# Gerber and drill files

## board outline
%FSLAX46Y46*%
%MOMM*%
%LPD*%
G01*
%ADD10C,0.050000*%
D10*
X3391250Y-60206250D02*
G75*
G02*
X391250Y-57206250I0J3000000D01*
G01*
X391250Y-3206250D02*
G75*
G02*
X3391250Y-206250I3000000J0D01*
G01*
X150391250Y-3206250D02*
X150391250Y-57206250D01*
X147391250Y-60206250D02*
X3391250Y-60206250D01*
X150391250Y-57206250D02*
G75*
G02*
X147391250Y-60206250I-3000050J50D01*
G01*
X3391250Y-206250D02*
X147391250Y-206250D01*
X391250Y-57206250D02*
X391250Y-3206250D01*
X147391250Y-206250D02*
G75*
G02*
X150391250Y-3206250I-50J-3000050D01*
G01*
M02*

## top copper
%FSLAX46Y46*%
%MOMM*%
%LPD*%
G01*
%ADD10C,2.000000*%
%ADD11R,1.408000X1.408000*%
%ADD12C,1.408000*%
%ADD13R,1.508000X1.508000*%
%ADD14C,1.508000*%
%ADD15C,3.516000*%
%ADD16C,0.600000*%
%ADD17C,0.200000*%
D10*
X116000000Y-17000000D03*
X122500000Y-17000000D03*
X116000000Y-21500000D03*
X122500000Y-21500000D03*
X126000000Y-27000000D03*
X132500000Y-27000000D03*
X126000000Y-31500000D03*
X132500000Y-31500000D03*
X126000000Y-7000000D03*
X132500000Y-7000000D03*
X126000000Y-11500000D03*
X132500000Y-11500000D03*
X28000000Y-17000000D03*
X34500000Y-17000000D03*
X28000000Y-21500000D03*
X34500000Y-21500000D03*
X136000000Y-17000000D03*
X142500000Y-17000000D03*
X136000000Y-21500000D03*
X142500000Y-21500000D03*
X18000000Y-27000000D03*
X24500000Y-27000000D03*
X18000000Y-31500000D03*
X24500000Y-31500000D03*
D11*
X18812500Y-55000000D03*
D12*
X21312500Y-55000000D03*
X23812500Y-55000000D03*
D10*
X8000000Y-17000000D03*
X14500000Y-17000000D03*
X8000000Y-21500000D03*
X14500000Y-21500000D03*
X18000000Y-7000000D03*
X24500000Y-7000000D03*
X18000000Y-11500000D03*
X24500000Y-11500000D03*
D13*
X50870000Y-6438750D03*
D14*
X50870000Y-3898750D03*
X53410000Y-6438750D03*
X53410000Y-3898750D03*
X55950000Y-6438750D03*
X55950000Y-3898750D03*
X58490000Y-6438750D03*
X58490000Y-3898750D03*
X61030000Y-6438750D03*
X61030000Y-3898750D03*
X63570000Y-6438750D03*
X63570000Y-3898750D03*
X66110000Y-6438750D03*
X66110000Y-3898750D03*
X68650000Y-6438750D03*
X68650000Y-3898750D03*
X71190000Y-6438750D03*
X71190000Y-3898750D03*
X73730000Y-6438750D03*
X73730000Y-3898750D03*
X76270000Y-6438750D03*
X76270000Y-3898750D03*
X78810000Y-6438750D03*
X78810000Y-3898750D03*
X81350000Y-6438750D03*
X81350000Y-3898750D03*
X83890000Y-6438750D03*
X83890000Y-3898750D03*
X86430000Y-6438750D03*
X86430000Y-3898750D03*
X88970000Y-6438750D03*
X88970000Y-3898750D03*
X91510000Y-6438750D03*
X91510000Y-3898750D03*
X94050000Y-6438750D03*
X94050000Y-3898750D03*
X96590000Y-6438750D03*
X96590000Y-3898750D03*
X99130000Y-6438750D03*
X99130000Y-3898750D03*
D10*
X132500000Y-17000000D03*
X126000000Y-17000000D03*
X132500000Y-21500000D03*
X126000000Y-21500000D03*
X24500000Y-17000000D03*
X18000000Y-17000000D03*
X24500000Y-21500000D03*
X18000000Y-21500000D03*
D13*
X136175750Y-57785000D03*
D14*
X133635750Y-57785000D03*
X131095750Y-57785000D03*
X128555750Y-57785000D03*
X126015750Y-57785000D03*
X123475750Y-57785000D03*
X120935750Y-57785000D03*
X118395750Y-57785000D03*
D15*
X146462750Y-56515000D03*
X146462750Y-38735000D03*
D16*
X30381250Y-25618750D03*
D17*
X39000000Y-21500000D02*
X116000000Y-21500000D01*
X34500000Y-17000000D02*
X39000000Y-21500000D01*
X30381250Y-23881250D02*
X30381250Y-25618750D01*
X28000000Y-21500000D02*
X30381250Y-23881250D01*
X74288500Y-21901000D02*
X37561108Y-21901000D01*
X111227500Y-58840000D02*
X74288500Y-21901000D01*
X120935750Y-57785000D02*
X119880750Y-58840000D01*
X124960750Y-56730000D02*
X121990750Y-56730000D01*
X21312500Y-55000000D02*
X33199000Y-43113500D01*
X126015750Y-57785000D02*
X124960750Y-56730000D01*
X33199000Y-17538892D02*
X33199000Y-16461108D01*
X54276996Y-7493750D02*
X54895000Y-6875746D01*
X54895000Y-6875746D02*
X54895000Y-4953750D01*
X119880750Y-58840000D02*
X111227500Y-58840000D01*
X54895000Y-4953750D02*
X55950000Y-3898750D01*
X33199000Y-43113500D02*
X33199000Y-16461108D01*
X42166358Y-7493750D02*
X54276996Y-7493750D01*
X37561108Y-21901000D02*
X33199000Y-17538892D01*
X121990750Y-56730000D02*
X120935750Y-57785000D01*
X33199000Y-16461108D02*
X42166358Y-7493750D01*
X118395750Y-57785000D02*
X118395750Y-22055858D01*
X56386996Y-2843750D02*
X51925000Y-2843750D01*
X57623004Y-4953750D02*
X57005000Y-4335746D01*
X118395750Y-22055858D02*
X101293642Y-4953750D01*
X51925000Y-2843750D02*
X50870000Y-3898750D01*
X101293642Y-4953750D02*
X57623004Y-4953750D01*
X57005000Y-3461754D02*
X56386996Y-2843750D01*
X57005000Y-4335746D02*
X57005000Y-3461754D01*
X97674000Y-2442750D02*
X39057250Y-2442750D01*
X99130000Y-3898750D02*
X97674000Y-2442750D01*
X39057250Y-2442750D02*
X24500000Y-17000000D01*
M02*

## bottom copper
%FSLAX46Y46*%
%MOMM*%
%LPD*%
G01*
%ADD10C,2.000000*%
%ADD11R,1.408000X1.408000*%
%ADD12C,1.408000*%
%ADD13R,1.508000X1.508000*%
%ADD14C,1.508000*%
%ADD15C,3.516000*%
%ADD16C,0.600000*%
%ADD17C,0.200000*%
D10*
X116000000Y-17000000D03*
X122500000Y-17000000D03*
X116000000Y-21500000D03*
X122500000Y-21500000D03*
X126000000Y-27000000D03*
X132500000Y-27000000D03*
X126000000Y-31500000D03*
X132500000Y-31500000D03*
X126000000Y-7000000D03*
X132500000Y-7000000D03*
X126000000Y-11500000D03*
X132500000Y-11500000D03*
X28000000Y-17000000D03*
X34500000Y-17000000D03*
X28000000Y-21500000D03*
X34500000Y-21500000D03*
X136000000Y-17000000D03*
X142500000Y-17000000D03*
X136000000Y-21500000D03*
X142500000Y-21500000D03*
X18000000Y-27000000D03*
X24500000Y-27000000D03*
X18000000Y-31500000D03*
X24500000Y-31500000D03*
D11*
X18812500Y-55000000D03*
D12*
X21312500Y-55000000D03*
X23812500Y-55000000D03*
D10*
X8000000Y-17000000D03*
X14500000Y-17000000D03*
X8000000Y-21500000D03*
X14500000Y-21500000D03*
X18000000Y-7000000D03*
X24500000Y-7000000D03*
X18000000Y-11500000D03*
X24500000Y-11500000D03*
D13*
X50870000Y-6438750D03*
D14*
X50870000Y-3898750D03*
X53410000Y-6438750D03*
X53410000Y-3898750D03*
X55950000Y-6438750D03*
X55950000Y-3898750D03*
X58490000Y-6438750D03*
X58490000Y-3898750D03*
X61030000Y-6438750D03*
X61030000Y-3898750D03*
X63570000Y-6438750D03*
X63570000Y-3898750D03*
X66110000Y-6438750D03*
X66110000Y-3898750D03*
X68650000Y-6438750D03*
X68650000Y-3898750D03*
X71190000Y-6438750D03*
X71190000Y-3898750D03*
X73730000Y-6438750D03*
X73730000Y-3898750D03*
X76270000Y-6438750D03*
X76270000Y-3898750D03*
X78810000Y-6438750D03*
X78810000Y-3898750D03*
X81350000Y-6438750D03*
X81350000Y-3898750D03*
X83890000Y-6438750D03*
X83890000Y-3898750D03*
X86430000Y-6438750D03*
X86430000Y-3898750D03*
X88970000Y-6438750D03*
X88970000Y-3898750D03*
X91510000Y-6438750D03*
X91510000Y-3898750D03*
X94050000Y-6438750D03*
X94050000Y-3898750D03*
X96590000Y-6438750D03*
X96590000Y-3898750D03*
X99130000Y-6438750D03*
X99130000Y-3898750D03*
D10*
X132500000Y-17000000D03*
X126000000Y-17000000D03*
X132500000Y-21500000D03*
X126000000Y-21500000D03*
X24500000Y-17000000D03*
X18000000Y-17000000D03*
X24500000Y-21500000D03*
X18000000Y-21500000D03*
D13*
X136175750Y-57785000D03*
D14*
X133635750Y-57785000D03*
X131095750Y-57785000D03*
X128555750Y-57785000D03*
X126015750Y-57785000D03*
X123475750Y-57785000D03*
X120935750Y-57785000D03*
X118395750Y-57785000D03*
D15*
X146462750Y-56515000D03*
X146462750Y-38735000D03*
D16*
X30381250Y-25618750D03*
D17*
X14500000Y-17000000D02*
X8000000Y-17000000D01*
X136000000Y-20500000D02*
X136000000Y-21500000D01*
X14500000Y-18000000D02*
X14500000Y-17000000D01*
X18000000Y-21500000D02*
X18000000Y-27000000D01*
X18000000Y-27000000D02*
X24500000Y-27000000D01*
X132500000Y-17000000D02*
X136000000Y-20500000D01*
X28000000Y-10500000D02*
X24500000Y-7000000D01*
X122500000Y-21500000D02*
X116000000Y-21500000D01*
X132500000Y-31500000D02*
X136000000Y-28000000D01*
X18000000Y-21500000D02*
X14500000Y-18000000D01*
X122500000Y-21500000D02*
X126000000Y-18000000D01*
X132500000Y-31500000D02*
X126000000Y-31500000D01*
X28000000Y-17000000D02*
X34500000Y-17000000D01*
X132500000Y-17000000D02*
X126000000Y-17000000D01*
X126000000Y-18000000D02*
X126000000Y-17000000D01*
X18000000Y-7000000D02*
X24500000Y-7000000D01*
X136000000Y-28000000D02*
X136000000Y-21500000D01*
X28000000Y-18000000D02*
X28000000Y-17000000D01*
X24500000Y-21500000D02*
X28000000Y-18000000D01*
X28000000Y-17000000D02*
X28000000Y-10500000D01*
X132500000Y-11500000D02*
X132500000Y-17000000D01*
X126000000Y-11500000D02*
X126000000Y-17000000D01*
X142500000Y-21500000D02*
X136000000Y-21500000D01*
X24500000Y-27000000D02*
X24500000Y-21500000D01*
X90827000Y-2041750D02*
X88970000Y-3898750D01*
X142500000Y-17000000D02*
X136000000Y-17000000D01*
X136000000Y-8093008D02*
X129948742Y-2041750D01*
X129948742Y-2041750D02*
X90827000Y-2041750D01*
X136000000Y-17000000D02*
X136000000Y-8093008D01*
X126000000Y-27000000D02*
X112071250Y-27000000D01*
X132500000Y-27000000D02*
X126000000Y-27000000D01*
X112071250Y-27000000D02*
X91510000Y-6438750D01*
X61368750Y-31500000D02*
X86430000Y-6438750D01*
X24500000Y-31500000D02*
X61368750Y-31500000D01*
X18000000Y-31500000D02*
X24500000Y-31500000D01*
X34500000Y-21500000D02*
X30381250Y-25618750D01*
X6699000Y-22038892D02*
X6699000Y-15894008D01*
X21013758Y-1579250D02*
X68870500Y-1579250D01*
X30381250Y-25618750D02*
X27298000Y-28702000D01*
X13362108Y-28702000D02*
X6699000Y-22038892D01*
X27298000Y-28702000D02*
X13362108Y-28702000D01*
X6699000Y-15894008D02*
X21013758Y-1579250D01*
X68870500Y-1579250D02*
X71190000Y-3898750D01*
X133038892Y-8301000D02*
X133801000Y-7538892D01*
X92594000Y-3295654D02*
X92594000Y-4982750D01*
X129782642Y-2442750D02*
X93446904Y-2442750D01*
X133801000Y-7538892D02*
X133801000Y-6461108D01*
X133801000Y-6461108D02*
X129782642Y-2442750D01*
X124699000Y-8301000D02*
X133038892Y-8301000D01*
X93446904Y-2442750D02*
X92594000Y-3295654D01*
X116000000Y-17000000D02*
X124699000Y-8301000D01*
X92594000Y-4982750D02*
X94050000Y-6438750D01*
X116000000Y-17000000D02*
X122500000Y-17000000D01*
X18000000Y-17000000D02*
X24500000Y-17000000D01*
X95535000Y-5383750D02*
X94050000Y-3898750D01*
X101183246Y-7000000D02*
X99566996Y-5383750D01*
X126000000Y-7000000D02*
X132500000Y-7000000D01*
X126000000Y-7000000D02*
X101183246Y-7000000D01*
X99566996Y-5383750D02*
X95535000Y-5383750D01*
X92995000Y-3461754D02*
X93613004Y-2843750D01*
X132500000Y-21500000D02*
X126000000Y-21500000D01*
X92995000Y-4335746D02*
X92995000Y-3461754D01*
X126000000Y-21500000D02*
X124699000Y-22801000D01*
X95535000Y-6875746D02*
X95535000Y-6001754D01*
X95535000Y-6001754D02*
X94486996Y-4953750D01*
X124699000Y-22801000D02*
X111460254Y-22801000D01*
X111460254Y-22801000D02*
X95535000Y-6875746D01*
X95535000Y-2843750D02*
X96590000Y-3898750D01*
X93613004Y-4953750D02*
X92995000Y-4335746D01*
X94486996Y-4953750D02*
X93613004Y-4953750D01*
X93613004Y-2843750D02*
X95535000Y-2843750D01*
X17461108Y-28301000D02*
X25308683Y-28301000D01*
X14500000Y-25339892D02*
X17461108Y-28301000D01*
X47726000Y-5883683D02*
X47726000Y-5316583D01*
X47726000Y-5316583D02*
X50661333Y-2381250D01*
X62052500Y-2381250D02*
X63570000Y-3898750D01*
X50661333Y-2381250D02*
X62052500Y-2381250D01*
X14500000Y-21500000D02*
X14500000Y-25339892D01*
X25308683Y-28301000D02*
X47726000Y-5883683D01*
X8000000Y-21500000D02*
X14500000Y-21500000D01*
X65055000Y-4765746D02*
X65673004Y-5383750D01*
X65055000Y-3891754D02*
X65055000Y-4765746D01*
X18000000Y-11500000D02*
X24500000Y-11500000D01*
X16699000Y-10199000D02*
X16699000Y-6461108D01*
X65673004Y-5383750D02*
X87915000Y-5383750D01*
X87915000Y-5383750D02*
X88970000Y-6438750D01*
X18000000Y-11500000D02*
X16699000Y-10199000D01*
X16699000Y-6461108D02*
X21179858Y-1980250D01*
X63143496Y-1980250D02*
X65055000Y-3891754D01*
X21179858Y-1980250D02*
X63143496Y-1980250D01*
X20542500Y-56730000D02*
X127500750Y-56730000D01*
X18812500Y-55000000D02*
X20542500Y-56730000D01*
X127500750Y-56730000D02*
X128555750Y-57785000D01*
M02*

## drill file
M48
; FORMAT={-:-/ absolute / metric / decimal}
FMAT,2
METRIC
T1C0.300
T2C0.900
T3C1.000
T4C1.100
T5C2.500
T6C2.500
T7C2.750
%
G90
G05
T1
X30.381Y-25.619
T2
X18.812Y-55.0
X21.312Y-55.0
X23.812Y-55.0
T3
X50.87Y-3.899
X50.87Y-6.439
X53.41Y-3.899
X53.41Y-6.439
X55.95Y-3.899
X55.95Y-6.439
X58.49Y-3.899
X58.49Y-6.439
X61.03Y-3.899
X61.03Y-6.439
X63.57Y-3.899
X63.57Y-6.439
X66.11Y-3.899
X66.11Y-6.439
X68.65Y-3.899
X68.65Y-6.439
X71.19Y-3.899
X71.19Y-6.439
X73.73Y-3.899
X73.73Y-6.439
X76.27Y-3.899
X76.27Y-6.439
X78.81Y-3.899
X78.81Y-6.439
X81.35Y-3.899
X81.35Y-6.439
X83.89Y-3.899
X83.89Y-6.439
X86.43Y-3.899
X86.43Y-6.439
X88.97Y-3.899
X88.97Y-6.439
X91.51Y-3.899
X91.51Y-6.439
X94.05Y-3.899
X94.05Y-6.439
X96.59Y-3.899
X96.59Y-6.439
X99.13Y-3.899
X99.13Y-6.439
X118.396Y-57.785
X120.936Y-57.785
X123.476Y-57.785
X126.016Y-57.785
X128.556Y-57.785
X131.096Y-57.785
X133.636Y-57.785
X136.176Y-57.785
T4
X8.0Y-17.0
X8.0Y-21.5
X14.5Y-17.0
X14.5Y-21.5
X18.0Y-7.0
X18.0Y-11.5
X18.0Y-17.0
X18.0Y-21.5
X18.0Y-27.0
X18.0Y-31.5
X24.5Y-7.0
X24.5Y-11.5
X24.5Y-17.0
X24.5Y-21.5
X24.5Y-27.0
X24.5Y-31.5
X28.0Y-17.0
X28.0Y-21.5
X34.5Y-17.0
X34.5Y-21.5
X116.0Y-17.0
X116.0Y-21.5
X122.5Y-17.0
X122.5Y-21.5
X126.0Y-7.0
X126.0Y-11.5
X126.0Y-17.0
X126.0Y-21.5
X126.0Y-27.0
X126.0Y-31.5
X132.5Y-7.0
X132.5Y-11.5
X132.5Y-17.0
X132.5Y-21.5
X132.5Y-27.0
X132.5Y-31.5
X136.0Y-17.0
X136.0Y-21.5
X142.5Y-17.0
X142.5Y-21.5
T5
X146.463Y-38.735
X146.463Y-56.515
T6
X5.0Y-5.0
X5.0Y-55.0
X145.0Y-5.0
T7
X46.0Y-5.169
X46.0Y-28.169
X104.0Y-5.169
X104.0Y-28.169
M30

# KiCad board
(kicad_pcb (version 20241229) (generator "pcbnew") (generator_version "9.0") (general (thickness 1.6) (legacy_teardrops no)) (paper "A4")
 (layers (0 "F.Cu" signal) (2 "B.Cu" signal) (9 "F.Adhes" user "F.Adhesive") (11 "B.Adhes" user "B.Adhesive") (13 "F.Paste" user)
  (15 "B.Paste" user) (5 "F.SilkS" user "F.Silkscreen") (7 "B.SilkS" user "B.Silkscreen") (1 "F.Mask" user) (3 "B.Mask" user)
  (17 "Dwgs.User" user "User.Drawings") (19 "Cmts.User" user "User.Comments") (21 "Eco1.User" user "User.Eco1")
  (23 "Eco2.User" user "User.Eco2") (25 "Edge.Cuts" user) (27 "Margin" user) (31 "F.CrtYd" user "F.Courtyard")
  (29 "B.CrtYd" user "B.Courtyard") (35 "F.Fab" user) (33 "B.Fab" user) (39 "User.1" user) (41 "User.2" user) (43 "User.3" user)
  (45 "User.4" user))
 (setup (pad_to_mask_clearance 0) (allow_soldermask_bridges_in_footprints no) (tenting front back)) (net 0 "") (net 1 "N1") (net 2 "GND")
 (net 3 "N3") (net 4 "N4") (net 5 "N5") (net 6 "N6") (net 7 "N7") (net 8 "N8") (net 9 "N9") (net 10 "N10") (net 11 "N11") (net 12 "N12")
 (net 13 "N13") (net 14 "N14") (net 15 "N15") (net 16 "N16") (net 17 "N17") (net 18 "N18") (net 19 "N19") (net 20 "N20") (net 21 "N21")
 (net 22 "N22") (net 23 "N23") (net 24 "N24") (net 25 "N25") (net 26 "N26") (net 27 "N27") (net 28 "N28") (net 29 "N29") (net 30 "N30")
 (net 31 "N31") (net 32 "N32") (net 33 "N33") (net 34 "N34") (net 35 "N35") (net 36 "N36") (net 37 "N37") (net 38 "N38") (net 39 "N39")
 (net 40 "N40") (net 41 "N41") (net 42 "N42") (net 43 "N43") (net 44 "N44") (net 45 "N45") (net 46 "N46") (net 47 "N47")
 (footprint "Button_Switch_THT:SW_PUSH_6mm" (layer "F.Cu") (at 116 17)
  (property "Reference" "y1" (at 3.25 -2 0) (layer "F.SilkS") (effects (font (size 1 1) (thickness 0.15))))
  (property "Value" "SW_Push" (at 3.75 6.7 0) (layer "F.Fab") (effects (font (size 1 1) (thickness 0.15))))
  (pad "1" thru_hole circle (at 0 0 90) (size 2 2) (drill 1.1) (layers "*.Cu" "*.Mask") (remove_unused_layers no) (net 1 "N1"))
  (pad "1" thru_hole circle (at 6.5 0 90) (size 2 2) (drill 1.1) (layers "*.Cu" "*.Mask") (remove_unused_layers no) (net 1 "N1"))
  (pad "2" thru_hole circle (at 0 4.5 90) (size 2 2) (drill 1.1) (layers "*.Cu" "*.Mask") (remove_unused_layers no) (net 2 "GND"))
  (pad "2" thru_hole circle (at 6.5 4.5 90) (size 2 2) (drill 1.1) (layers "*.Cu" "*.Mask") (remove_unused_layers no) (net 2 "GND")))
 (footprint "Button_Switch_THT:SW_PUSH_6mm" (layer "F.Cu") (at 126 27)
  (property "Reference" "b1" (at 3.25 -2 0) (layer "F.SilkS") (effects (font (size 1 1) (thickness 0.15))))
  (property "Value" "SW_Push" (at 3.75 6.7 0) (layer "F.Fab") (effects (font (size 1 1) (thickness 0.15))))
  (pad "1" thru_hole circle (at 0 0 90) (size 2 2) (drill 1.1) (layers "*.Cu" "*.Mask") (remove_unused_layers no) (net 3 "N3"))
  (pad "1" thru_hole circle (at 6.5 0 90) (size 2 2) (drill 1.1) (layers "*.Cu" "*.Mask") (remove_unused_layers no) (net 3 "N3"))
  (pad "2" thru_hole circle (at 0 4.5 90) (size 2 2) (drill 1.1) (layers "*.Cu" "*.Mask") (remove_unused_layers no) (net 2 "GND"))
  (pad "2" thru_hole circle (at 6.5 4.5 90) (size 2 2) (drill 1.1) (layers "*.Cu" "*.Mask") (remove_unused_layers no) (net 2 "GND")))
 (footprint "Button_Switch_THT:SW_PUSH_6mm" (layer "F.Cu") (at 126 7)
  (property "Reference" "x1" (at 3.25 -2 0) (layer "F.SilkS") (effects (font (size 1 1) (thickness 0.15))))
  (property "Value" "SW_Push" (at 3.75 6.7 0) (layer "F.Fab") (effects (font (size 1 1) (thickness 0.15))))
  (pad "1" thru_hole circle (at 0 0 90) (size 2 2) (drill 1.1) (layers "*.Cu" "*.Mask") (remove_unused_layers no) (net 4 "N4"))
  (pad "1" thru_hole circle (at 6.5 0 90) (size 2 2) (drill 1.1) (layers "*.Cu" "*.Mask") (remove_unused_layers no) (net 4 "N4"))
  (pad "2" thru_hole circle (at 0 4.5 90) (size 2 2) (drill 1.1) (layers "*.Cu" "*.Mask") (remove_unused_layers no) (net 2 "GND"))
  (pad "2" thru_hole circle (at 6.5 4.5 90) (size 2 2) (drill 1.1) (layers "*.Cu" "*.Mask") (remove_unused_layers no) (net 2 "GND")))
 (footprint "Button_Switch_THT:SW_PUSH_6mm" (layer "F.Cu") (at 28 17)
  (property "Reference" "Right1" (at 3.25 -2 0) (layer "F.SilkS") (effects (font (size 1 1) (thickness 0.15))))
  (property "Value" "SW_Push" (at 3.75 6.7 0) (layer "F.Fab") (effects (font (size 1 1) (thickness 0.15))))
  (pad "1" thru_hole circle (at 0 0 90) (size 2 2) (drill 1.1) (layers "*.Cu" "*.Mask") (remove_unused_layers no) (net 2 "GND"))
  (pad "1" thru_hole circle (at 6.5 0 90) (size 2 2) (drill 1.1) (layers "*.Cu" "*.Mask") (remove_unused_layers no) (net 2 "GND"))
  (pad "2" thru_hole circle (at 0 4.5 90) (size 2 2) (drill 1.1) (layers "*.Cu" "*.Mask") (remove_unused_layers no) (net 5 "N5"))
  (pad "2" thru_hole circle (at 6.5 4.5 90) (size 2 2) (drill 1.1) (layers "*.Cu" "*.Mask") (remove_unused_layers no) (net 5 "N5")))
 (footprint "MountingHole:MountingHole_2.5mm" (layer "F.Cu") (at 145 5)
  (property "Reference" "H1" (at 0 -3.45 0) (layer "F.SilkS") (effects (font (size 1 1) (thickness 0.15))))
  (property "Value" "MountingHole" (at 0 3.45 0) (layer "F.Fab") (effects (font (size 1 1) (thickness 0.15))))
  (pad "" np_thru_hole circle (at 0 0) (size 2.5 2.5) (drill 2.5) (layers "*.Cu" "*.Mask")))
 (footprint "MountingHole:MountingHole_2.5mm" (layer "F.Cu") (at 5 5)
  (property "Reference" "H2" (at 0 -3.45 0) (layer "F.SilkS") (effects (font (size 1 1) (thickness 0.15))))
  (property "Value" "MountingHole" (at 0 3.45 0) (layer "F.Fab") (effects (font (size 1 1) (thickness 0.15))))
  (pad "" np_thru_hole circle (at 0 0) (size 2.5 2.5) (drill 2.5) (layers "*.Cu" "*.Mask")))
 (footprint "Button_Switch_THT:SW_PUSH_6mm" (layer "F.Cu") (at 136 17)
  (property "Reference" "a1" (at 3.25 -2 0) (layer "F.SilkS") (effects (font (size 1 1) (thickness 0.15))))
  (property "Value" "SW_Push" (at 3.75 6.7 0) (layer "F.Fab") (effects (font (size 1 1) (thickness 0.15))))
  (pad "1" thru_hole circle (at 0 0 90) (size 2 2) (drill 1.1) (layers "*.Cu" "*.Mask") (remove_unused_layers no) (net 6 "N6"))
  (pad "1" thru_hole circle (at 6.5 0 90) (size 2 2) (drill 1.1) (layers "*.Cu" "*.Mask") (remove_unused_layers no) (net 6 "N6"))
  (pad "2" thru_hole circle (at 0 4.5 90) (size 2 2) (drill 1.1) (layers "*.Cu" "*.Mask") (remove_unused_layers no) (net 2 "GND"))
  (pad "2" thru_hole circle (at 6.5 4.5 90) (size 2 2) (drill 1.1) (layers "*.Cu" "*.Mask") (remove_unused_layers no) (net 2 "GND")))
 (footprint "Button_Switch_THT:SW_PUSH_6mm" (layer "F.Cu") (at 18 27)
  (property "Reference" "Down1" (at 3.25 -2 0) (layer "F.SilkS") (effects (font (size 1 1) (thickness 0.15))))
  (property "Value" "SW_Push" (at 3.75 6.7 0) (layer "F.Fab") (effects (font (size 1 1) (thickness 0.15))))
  (pad "1" thru_hole circle (at 0 0 90) (size 2 2) (drill 1.1) (layers "*.Cu" "*.Mask") (remove_unused_layers no) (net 2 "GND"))
  (pad "1" thru_hole circle (at 6.5 0 90) (size 2 2) (drill 1.1) (layers "*.Cu" "*.Mask") (remove_unused_layers no) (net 2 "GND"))
  (pad "2" thru_hole circle (at 0 4.5 90) (size 2 2) (drill 1.1) (layers "*.Cu" "*.Mask") (remove_unused_layers no) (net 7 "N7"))
  (pad "2" thru_hole circle (at 6.5 4.5 90) (size 2 2) (drill 1.1) (layers "*.Cu" "*.Mask") (remove_unused_layers no) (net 7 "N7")))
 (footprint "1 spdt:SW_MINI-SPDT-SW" (layer "F.Cu") (at 21.3125 55)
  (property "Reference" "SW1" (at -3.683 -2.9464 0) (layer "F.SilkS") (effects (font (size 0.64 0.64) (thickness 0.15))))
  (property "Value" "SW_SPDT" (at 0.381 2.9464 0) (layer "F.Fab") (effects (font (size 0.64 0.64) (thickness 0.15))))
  (pad "1" thru_hole rect (at -2.5 0) (size 1.408 1.408) (drill 0.9) (layers "*.Cu" "*.Mask") (remove_unused_layers no) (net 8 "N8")
   (solder_mask_margin 0.102))
  (pad "2" thru_hole circle (at 0 0) (size 1.408 1.408) (drill 0.9) (layers "*.Cu" "*.Mask") (remove_unused_layers no) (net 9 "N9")
   (solder_mask_margin 0.102))
  (pad "3" thru_hole circle (at 2.5 0) (size 1.408 1.408) (drill 0.9) (layers "*.Cu" "*.Mask") (remove_unused_layers no) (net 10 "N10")
   (solder_mask_margin 0.102)))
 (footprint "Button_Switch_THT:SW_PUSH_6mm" (layer "F.Cu") (at 8 17)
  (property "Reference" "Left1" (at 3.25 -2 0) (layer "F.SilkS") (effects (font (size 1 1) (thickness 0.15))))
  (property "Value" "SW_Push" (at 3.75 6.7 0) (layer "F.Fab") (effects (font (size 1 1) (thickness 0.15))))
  (pad "1" thru_hole circle (at 0 0 90) (size 2 2) (drill 1.1) (layers "*.Cu" "*.Mask") (remove_unused_layers no) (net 2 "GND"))
  (pad "1" thru_hole circle (at 6.5 0 90) (size 2 2) (drill 1.1) (layers "*.Cu" "*.Mask") (remove_unused_layers no) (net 2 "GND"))
  (pad "2" thru_hole circle (at 0 4.5 90) (size 2 2) (drill 1.1) (layers "*.Cu" "*.Mask") (remove_unused_layers no) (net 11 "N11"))
  (pad "2" thru_hole circle (at 6.5 4.5 90) (size 2 2) (drill 1.1) (layers "*.Cu" "*.Mask") (remove_unused_layers no) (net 11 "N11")))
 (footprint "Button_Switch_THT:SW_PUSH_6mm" (layer "F.Cu") (at 18 7)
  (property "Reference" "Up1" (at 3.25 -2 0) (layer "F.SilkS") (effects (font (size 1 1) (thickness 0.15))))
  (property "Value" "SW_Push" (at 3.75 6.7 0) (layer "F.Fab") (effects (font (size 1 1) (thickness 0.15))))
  (pad "1" thru_hole circle (at 0 0 90) (size 2 2) (drill 1.1) (layers "*.Cu" "*.Mask") (remove_unused_layers no) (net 2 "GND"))
  (pad "1" thru_hole circle (at 6.5 0 90) (size 2 2) (drill 1.1) (layers "*.Cu" "*.Mask") (remove_unused_layers no) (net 2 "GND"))
  (pad "2" thru_hole circle (at 0 4.5 90) (size 2 2) (drill 1.1) (layers "*.Cu" "*.Mask") (remove_unused_layers no) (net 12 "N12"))
  (pad "2" thru_hole circle (at 6.5 4.5 90) (size 2 2) (drill 1.1) (layers "*.Cu" "*.Mask") (remove_unused_layers no) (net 12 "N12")))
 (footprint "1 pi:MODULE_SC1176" (layer "F.Cu") (at 75 16.66875)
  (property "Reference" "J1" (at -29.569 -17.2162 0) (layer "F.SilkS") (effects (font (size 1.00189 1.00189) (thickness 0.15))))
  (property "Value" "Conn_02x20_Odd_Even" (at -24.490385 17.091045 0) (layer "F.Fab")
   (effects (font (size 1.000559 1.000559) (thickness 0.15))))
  (pad "" np_thru_hole circle (at -29 -11.5) (size 2.75 2.75) (drill 2.75) (layers "*.Cu" "*.Mask"))
  (pad "" np_thru_hole circle (at -29 11.5) (size 2.75 2.75) (drill 2.75) (layers "*.Cu" "*.Mask"))
  (pad "" np_thru_hole circle (at 29 -11.5) (size 2.75 2.75) (drill 2.75) (layers "*.Cu" "*.Mask"))
  (pad "" np_thru_hole circle (at 29 11.5) (size 2.75 2.75) (drill 2.75) (layers "*.Cu" "*.Mask"))
  (pad "1" thru_hole rect (at -24.13 -10.23) (size 1.508 1.508) (drill 1) (layers "*.Cu" "*.Mask") (remove_unused_layers no) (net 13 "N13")
   (solder_mask_margin 0.102))
  (pad "2" thru_hole circle (at -24.13 -12.77) (size 1.508 1.508) (drill 1) (layers "*.Cu" "*.Mask") (remove_unused_layers no)
   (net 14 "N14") (solder_mask_margin 0.102))
  (pad "3" thru_hole circle (at -21.59 -10.23) (size 1.508 1.508) (drill 1) (layers "*.Cu" "*.Mask") (remove_unused_layers no)
   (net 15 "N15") (solder_mask_margin 0.102))
  (pad "4" thru_hole circle (at -21.59 -12.77) (size 1.508 1.508) (drill 1) (layers "*.Cu" "*.Mask") (remove_unused_layers no)
   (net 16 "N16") (solder_mask_margin 0.102))
  (pad "5" thru_hole circle (at -19.05 -10.23) (size 1.508 1.508) (drill 1) (layers "*.Cu" "*.Mask") (remove_unused_layers no)
   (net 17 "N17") (solder_mask_margin 0.102))
  (pad "6" thru_hole circle (at -19.05 -12.77) (size 1.508 1.508) (drill 1) (layers "*.Cu" "*.Mask") (remove_unused_layers no) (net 9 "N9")
   (solder_mask_margin 0.102))
  (pad "7" thru_hole circle (at -16.51 -10.23) (size 1.508 1.508) (drill 1) (layers "*.Cu" "*.Mask") (remove_unused_layers no)
   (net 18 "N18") (solder_mask_margin 0.102))
  (pad "8" thru_hole circle (at -16.51 -12.77) (size 1.508 1.508) (drill 1) (layers "*.Cu" "*.Mask") (remove_unused_layers no)
   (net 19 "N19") (solder_mask_margin 0.102))
  (pad "9" thru_hole circle (at -13.97 -10.23) (size 1.508 1.508) (drill 1) (layers "*.Cu" "*.Mask") (remove_unused_layers no)
   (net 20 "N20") (solder_mask_margin 0.102))
  (pad "10" thru_hole circle (at -13.97 -12.77) (size 1.508 1.508) (drill 1) (layers "*.Cu" "*.Mask") (remove_unused_layers no)
   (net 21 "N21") (solder_mask_margin 0.102))
  (pad "11" thru_hole circle (at -11.43 -10.23) (size 1.508 1.508) (drill 1) (layers "*.Cu" "*.Mask") (remove_unused_layers no)
   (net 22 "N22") (solder_mask_margin 0.102))
  (pad "12" thru_hole circle (at -11.43 -12.77) (size 1.508 1.508) (drill 1) (layers "*.Cu" "*.Mask") (remove_unused_layers no)
   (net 11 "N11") (solder_mask_margin 0.102))
  (pad "13" thru_hole circle (at -8.89 -10.23) (size 1.508 1.508) (drill 1) (layers "*.Cu" "*.Mask") (remove_unused_layers no)
   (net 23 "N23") (solder_mask_margin 0.102))
  (pad "14" thru_hole circle (at -8.89 -12.77) (size 1.508 1.508) (drill 1) (layers "*.Cu" "*.Mask") (remove_unused_layers no)
   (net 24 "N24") (solder_mask_margin 0.102))
  (pad "15" thru_hole circle (at -6.35 -10.23) (size 1.508 1.508) (drill 1) (layers "*.Cu" "*.Mask") (remove_unused_layers no)
   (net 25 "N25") (solder_mask_margin 0.102))
  (pad "16" thru_hole circle (at -6.35 -12.77) (size 1.508 1.508) (drill 1) (layers "*.Cu" "*.Mask") (remove_unused_layers no)
   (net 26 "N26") (solder_mask_margin 0.102))
  (pad "17" thru_hole circle (at -3.81 -10.23) (size 1.508 1.508) (drill 1) (layers "*.Cu" "*.Mask") (remove_unused_layers no)
   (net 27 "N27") (solder_mask_margin 0.102))
  (pad "18" thru_hole circle (at -3.81 -12.77) (size 1.508 1.508) (drill 1) (layers "*.Cu" "*.Mask") (remove_unused_layers no) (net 5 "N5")
   (solder_mask_margin 0.102))
  (pad "19" thru_hole circle (at -1.27 -10.23) (size 1.508 1.508) (drill 1) (layers "*.Cu" "*.Mask") (remove_unused_layers no)
   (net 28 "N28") (solder_mask_margin 0.102))
  (pad "20" thru_hole circle (at -1.27 -12.77) (size 1.508 1.508) (drill 1) (layers "*.Cu" "*.Mask") (remove_unused_layers no)
   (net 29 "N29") (solder_mask_margin 0.102))
  (pad "21" thru_hole circle (at 1.27 -10.23) (size 1.508 1.508) (drill 1) (layers "*.Cu" "*.Mask") (remove_unused_layers no) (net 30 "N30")
   (solder_mask_margin 0.102))
  (pad "22" thru_hole circle (at 1.27 -12.77) (size 1.508 1.508) (drill 1) (layers "*.Cu" "*.Mask") (remove_unused_layers no) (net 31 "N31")
   (solder_mask_margin 0.102))
  (pad "23" thru_hole circle (at 3.81 -10.23) (size 1.508 1.508) (drill 1) (layers "*.Cu" "*.Mask") (remove_unused_layers no) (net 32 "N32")
   (solder_mask_margin 0.102))
  (pad "24" thru_hole circle (at 3.81 -12.77) (size 1.508 1.508) (drill 1) (layers "*.Cu" "*.Mask") (remove_unused_layers no) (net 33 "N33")
   (solder_mask_margin 0.102))
  (pad "25" thru_hole circle (at 6.35 -10.23) (size 1.508 1.508) (drill 1) (layers "*.Cu" "*.Mask") (remove_unused_layers no) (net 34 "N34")
   (solder_mask_margin 0.102))
  (pad "26" thru_hole circle (at 6.35 -12.77) (size 1.508 1.508) (drill 1) (layers "*.Cu" "*.Mask") (remove_unused_layers no) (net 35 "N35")
   (solder_mask_margin 0.102))
  (pad "27" thru_hole circle (at 8.89 -10.23) (size 1.508 1.508) (drill 1) (layers "*.Cu" "*.Mask") (remove_unused_layers no) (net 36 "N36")
   (solder_mask_margin 0.102))
  (pad "28" thru_hole circle (at 8.89 -12.77) (size 1.508 1.508) (drill 1) (layers "*.Cu" "*.Mask") (remove_unused_layers no) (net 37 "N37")
   (solder_mask_margin 0.102))
  (pad "29" thru_hole circle (at 11.43 -10.23) (size 1.508 1.508) (drill 1) (layers "*.Cu" "*.Mask") (remove_unused_layers no) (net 7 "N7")
   (solder_mask_margin 0.102))
  (pad "30" thru_hole circle (at 11.43 -12.77) (size 1.508 1.508) (drill 1) (layers "*.Cu" "*.Mask") (remove_unused_layers no)
   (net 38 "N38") (solder_mask_margin 0.102))
  (pad "31" thru_hole circle (at 13.97 -10.23) (size 1.508 1.508) (drill 1) (layers "*.Cu" "*.Mask") (remove_unused_layers no)
   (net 12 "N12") (solder_mask_margin 0.102))
  (pad "32" thru_hole circle (at 13.97 -12.77) (size 1.508 1.508) (drill 1) (layers "*.Cu" "*.Mask") (remove_unused_layers no) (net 6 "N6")
   (solder_mask_margin 0.102))
  (pad "33" thru_hole circle (at 16.51 -10.23) (size 1.508 1.508) (drill 1) (layers "*.Cu" "*.Mask") (remove_unused_layers no) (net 3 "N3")
   (solder_mask_margin 0.102))
  (pad "34" thru_hole circle (at 16.51 -12.77) (size 1.508 1.508) (drill 1) (layers "*.Cu" "*.Mask") (remove_unused_layers no)
   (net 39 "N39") (solder_mask_margin 0.102))
  (pad "35" thru_hole circle (at 19.05 -10.23) (size 1.508 1.508) (drill 1) (layers "*.Cu" "*.Mask") (remove_unused_layers no) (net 1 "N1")
   (solder_mask_margin 0.102))
  (pad "36" thru_hole circle (at 19.05 -12.77) (size 1.508 1.508) (drill 1) (layers "*.Cu" "*.Mask") (remove_unused_layers no) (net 4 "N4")
   (solder_mask_margin 0.102))
  (pad "37" thru_hole circle (at 21.59 -10.23) (size 1.508 1.508) (drill 1) (layers "*.Cu" "*.Mask") (remove_unused_layers no)
   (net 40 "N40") (solder_mask_margin 0.102))
  (pad "38" thru_hole circle (at 21.59 -12.77) (size 1.508 1.508) (drill 1) (layers "*.Cu" "*.Mask") (remove_unused_layers no)
   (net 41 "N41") (solder_mask_margin 0.102))
  (pad "39" thru_hole circle (at 24.13 -10.23) (size 1.508 1.508) (drill 1) (layers "*.Cu" "*.Mask") (remove_unused_layers no)
   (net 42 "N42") (solder_mask_margin 0.102))
  (pad "40" thru_hole circle (at 24.13 -12.77) (size 1.508 1.508) (drill 1) (layers "*.Cu" "*.Mask") (remove_unused_layers no)
   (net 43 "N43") (solder_mask_margin 0.102)))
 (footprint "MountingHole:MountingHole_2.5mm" (layer "F.Cu") (at 5 55)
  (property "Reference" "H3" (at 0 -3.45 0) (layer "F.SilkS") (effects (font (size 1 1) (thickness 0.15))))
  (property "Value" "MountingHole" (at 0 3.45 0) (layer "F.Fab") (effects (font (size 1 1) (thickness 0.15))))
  (pad "" np_thru_hole circle (at 0 0) (size 2.5 2.5) (drill 2.5) (layers "*.Cu" "*.Mask")))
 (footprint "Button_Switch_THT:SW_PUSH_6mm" (layer "B.Cu") (at 132.5 17 180)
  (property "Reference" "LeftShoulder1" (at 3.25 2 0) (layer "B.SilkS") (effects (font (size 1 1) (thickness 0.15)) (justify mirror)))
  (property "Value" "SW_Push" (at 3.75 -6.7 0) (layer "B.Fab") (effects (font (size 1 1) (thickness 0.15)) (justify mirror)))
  (pad "1" thru_hole circle (at 0 0 90) (size 2 2) (drill 1.1) (layers "*.Cu" "*.Mask") (remove_unused_layers no) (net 2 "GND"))
  (pad "1" thru_hole circle (at 6.5 0 90) (size 2 2) (drill 1.1) (layers "*.Cu" "*.Mask") (remove_unused_layers no) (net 2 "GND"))
  (pad "2" thru_hole circle (at 0 -4.5 90) (size 2 2) (drill 1.1) (layers "*.Cu" "*.Mask") (remove_unused_layers no) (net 41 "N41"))
  (pad "2" thru_hole circle (at 6.5 -4.5 90) (size 2 2) (drill 1.1) (layers "*.Cu" "*.Mask") (remove_unused_layers no) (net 41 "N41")))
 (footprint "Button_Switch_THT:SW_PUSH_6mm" (layer "B.Cu") (at 24.5 17 180)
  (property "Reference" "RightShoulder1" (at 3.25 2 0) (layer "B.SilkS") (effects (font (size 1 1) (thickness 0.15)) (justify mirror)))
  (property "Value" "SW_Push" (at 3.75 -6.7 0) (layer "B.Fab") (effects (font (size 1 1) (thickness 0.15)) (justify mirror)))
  (pad "1" thru_hole circle (at 0 0 90) (size 2 2) (drill 1.1) (layers "*.Cu" "*.Mask") (remove_unused_layers no) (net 43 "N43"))
  (pad "1" thru_hole circle (at 6.5 0 90) (size 2 2) (drill 1.1) (layers "*.Cu" "*.Mask") (remove_unused_layers no) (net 43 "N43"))
  (pad "2" thru_hole circle (at 0 -4.5 90) (size 2 2) (drill 1.1) (layers "*.Cu" "*.Mask") (remove_unused_layers no) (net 2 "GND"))
  (pad "2" thru_hole circle (at 6.5 -4.5 90) (size 2 2) (drill 1.1) (layers "*.Cu" "*.Mask") (remove_unused_layers no) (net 2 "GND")))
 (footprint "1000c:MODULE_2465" (layer "B.Cu") (at 130.96875 47.625 180)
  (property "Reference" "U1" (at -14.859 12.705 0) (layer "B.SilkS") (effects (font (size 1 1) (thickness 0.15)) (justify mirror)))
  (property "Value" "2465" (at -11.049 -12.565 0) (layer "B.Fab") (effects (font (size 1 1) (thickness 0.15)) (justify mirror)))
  (pad "1" thru_hole rect (at -5.207 -10.16 180) (size 1.508 1.508) (drill 1) (layers "*.Cu" "*.Mask") (remove_unused_layers no)
   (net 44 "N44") (solder_mask_margin 0.102))
  (pad "2" thru_hole circle (at -2.667 -10.16 180) (size 1.508 1.508) (drill 1) (layers "*.Cu" "*.Mask") (remove_unused_layers no)
   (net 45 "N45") (solder_mask_margin 0.102))
  (pad "3" thru_hole circle (at -0.127 -10.16 180) (size 1.508 1.508) (drill 1) (layers "*.Cu" "*.Mask") (remove_unused_layers no)
   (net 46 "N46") (solder_mask_margin 0.102))
  (pad "4" thru_hole circle (at 2.413 -10.16 180) (size 1.508 1.508) (drill 1) (layers "*.Cu" "*.Mask") (remove_unused_layers no)
   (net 8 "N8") (solder_mask_margin 0.102))
  (pad "5" thru_hole circle (at 4.953 -10.16 180) (size 1.508 1.508) (drill 1) (layers "*.Cu" "*.Mask") (remove_unused_layers no)
   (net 9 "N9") (solder_mask_margin 0.102))
  (pad "6" thru_hole circle (at 7.493 -10.16 180) (size 1.508 1.508) (drill 1) (layers "*.Cu" "*.Mask") (remove_unused_layers no)
   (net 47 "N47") (solder_mask_margin 0.102))
  (pad "7" thru_hole circle (at 10.033 -10.16 180) (size 1.508 1.508) (drill 1) (layers "*.Cu" "*.Mask") (remove_unused_layers no)
   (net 9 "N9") (solder_mask_margin 0.102))
  (pad "8" thru_hole circle (at 12.573 -10.16 180) (size 1.508 1.508) (drill 1) (layers "*.Cu" "*.Mask") (remove_unused_layers no)
   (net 14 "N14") (solder_mask_margin 0.102))
  (pad "P1" thru_hole circle (at -15.494 -8.89 180) (size 3.516 3.516) (drill 2.5) (layers "*.Cu" "*.Mask") (remove_unused_layers no)
   (solder_mask_margin 0.102))
  (pad "P2" thru_hole circle (at -15.494 8.89 180) (size 3.516 3.516) (drill 2.5) (layers "*.Cu" "*.Mask") (remove_unused_layers no)
   (solder_mask_margin 0.102)))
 (gr_arc (start 3.39125 60.20625) (mid 1.26993 59.32757) (end 0.39125 57.20625) (stroke (width 0.05) (type default)) (layer "Edge.Cuts"))
 (gr_arc (start 0.39125 3.20625) (mid 1.26993 1.08493) (end 3.39125 0.20625) (stroke (width 0.05) (type default)) (layer "Edge.Cuts"))
 (gr_line (start 150.39125 3.20625) (end 150.39125 57.20625) (stroke (width 0.05) (type default)) (layer "Edge.Cuts"))
 (gr_line (start 147.39125 60.20625) (end 3.39125 60.20625) (stroke (width 0.05) (type default)) (layer "Edge.Cuts"))
 (gr_arc (start 150.39125 57.20625) (mid 149.51257 59.32757) (end 147.39125 60.20625) (stroke (width 0.05) (type default))
  (layer "Edge.Cuts"))
 (gr_line (start 3.39125 0.20625) (end 147.39125 0.20625) (stroke (width 0.05) (type default)) (layer "Edge.Cuts"))
 (gr_line (start 0.39125 57.20625) (end 0.39125 3.20625) (stroke (width 0.05) (type default)) (layer "Edge.Cuts"))
 (gr_arc (start 147.39125 0.20625) (mid 149.51257 1.08493) (end 150.39125 3.20625) (stroke (width 0.05) (type default)) (layer "Edge.Cuts"))
 (segment (start 39 21.5) (end 116 21.5) (width 0.2) (layer "F.Cu") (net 2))
 (segment (start 34.5 17) (end 39 21.5) (width 0.2) (layer "F.Cu") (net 2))
 (segment (start 14.5 17) (end 8 17) (width 0.2) (layer "B.Cu") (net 2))
 (segment (start 136 20.5) (end 136 21.5) (width 0.2) (layer "B.Cu") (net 2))
 (segment (start 14.5 18) (end 14.5 17) (width 0.2) (layer "B.Cu") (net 2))
 (segment (start 18 21.5) (end 18 27) (width 0.2) (layer "B.Cu") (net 2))
 (segment (start 18 27) (end 24.5 27) (width 0.2) (layer "B.Cu") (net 2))
 (segment (start 132.5 17) (end 136 20.5) (width 0.2) (layer "B.Cu") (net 2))
 (segment (start 28 10.5) (end 24.5 7) (width 0.2) (layer "B.Cu") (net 2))
 (segment (start 122.5 21.5) (end 116 21.5) (width 0.2) (layer "B.Cu") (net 2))
 (segment (start 132.5 31.5) (end 136 28) (width 0.2) (layer "B.Cu") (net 2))
 (segment (start 18 21.5) (end 14.5 18) (width 0.2) (layer "B.Cu") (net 2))
 (segment (start 122.5 21.5) (end 126 18) (width 0.2) (layer "B.Cu") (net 2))
 (segment (start 132.5 31.5) (end 126 31.5) (width 0.2) (layer "B.Cu") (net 2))
 (segment (start 28 17) (end 34.5 17) (width 0.2) (layer "B.Cu") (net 2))
 (segment (start 132.5 17) (end 126 17) (width 0.2) (layer "B.Cu") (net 2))
 (segment (start 126 18) (end 126 17) (width 0.2) (layer "B.Cu") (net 2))
 (segment (start 18 7) (end 24.5 7) (width 0.2) (layer "B.Cu") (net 2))
 (segment (start 136 28) (end 136 21.5) (width 0.2) (layer "B.Cu") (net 2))
 (segment (start 28 18) (end 28 17) (width 0.2) (layer "B.Cu") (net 2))
 (segment (start 24.5 21.5) (end 28 18) (width 0.2) (layer "B.Cu") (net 2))
 (segment (start 28 17) (end 28 10.5) (width 0.2) (layer "B.Cu") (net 2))
 (segment (start 132.5 11.5) (end 132.5 17) (width 0.2) (layer "B.Cu") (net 2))
 (segment (start 126 11.5) (end 126 17) (width 0.2) (layer "B.Cu") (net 2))
 (segment (start 142.5 21.5) (end 136 21.5) (width 0.2) (layer "B.Cu") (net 2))
 (segment (start 24.5 27) (end 24.5 21.5) (width 0.2) (layer "B.Cu") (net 2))
 (segment (start 90.827 2.04175) (end 88.97 3.89875) (width 0.2) (layer "B.Cu") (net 6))
 (segment (start 142.5 17) (end 136 17) (width 0.2) (layer "B.Cu") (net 6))
 (segment (start 136 8.093008) (end 129.948742 2.04175) (width 0.2) (layer "B.Cu") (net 6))
 (segment (start 129.948742 2.04175) (end 90.827 2.04175) (width 0.2) (layer "B.Cu") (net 6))
 (segment (start 136 17) (end 136 8.093008) (width 0.2) (layer "B.Cu") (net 6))
 (segment (start 126 27) (end 112.07125 27) (width 0.2) (layer "B.Cu") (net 3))
 (segment (start 132.5 27) (end 126 27) (width 0.2) (layer "B.Cu") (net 3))
 (segment (start 112.07125 27) (end 91.51 6.43875) (width 0.2) (layer "B.Cu") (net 3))
 (segment (start 61.36875 31.5) (end 86.43 6.43875) (width 0.2) (layer "B.Cu") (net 7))
 (segment (start 24.5 31.5) (end 61.36875 31.5) (width 0.2) (layer "B.Cu") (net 7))
 (segment (start 18 31.5) (end 24.5 31.5) (width 0.2) (layer "B.Cu") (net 7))
 (segment (start 30.38125 23.88125) (end 30.38125 25.61875) (width 0.2) (layer "F.Cu") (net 5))
 (segment (start 28 21.5) (end 30.38125 23.88125) (width 0.2) (layer "F.Cu") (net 5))
 (via (at 30.38125 25.61875) (size 0.6) (drill 0.3) (layers "F.Cu" "B.Cu") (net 5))
 (segment (start 34.5 21.5) (end 30.38125 25.61875) (width 0.2) (layer "B.Cu") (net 5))
 (segment (start 6.699 22.038892) (end 6.699 15.894008) (width 0.2) (layer "B.Cu") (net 5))
 (segment (start 21.013758 1.57925) (end 68.8705 1.57925) (width 0.2) (layer "B.Cu") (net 5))
 (segment (start 30.38125 25.61875) (end 27.298 28.702) (width 0.2) (layer "B.Cu") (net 5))
 (segment (start 13.362108 28.702) (end 6.699 22.038892) (width 0.2) (layer "B.Cu") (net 5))
 (segment (start 27.298 28.702) (end 13.362108 28.702) (width 0.2) (layer "B.Cu") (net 5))
 (segment (start 6.699 15.894008) (end 21.013758 1.57925) (width 0.2) (layer "B.Cu") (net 5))
 (segment (start 68.8705 1.57925) (end 71.19 3.89875) (width 0.2) (layer "B.Cu") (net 5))
 (segment (start 74.2885 21.901) (end 37.561108 21.901) (width 0.2) (layer "F.Cu") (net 9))
 (segment (start 111.2275 58.84) (end 74.2885 21.901) (width 0.2) (layer "F.Cu") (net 9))
 (segment (start 120.93575 57.785) (end 119.88075 58.84) (width 0.2) (layer "F.Cu") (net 9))
 (segment (start 124.96075 56.73) (end 121.99075 56.73) (width 0.2) (layer "F.Cu") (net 9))
 (segment (start 21.3125 55) (end 33.199 43.1135) (width 0.2) (layer "F.Cu") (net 9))
 (segment (start 126.01575 57.785) (end 124.96075 56.73) (width 0.2) (layer "F.Cu") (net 9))
 (segment (start 33.199 17.538892) (end 33.199 16.461108) (width 0.2) (layer "F.Cu") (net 9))
 (segment (start 54.276996 7.49375) (end 54.895 6.875746) (width 0.2) (layer "F.Cu") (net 9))
 (segment (start 54.895 6.875746) (end 54.895 4.95375) (width 0.2) (layer "F.Cu") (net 9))
 (segment (start 119.88075 58.84) (end 111.2275 58.84) (width 0.2) (layer "F.Cu") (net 9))
 (segment (start 54.895 4.95375) (end 55.95 3.89875) (width 0.2) (layer "F.Cu") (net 9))
 (segment (start 33.199 43.1135) (end 33.199 16.461108) (width 0.2) (layer "F.Cu") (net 9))
 (segment (start 42.166358 7.49375) (end 54.276996 7.49375) (width 0.2) (layer "F.Cu") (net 9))
 (segment (start 37.561108 21.901) (end 33.199 17.538892) (width 0.2) (layer "F.Cu") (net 9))
 (segment (start 121.99075 56.73) (end 120.93575 57.785) (width 0.2) (layer "F.Cu") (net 9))
 (segment (start 33.199 16.461108) (end 42.166358 7.49375) (width 0.2) (layer "F.Cu") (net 9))
 (segment (start 133.038892 8.301) (end 133.801 7.538892) (width 0.2) (layer "B.Cu") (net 1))
 (segment (start 92.594 3.295654) (end 92.594 4.98275) (width 0.2) (layer "B.Cu") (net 1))
 (segment (start 129.782642 2.44275) (end 93.446904 2.44275) (width 0.2) (layer "B.Cu") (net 1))
 (segment (start 133.801 7.538892) (end 133.801 6.461108) (width 0.2) (layer "B.Cu") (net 1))
 (segment (start 133.801 6.461108) (end 129.782642 2.44275) (width 0.2) (layer "B.Cu") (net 1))
 (segment (start 124.699 8.301) (end 133.038892 8.301) (width 0.2) (layer "B.Cu") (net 1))
 (segment (start 93.446904 2.44275) (end 92.594 3.295654) (width 0.2) (layer "B.Cu") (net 1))
 (segment (start 116 17) (end 124.699 8.301) (width 0.2) (layer "B.Cu") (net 1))
 (segment (start 92.594 4.98275) (end 94.05 6.43875) (width 0.2) (layer "B.Cu") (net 1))
 (segment (start 116 17) (end 122.5 17) (width 0.2) (layer "B.Cu") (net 1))
 (segment (start 118.39575 57.785) (end 118.39575 22.055858) (width 0.2) (layer "F.Cu") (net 14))
 (segment (start 56.386996 2.84375) (end 51.925 2.84375) (width 0.2) (layer "F.Cu") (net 14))
 (segment (start 57.623004 4.95375) (end 57.005 4.335746) (width 0.2) (layer "F.Cu") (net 14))
 (segment (start 118.39575 22.055858) (end 101.293642 4.95375) (width 0.2) (layer "F.Cu") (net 14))
 (segment (start 51.925 2.84375) (end 50.87 3.89875) (width 0.2) (layer "F.Cu") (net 14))
 (segment (start 101.293642 4.95375) (end 57.623004 4.95375) (width 0.2) (layer "F.Cu") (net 14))
 (segment (start 57.005 3.461754) (end 56.386996 2.84375) (width 0.2) (layer "F.Cu") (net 14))
 (segment (start 57.005 4.335746) (end 57.005 3.461754) (width 0.2) (layer "F.Cu") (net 14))
 (segment (start 97.674 2.44275) (end 39.05725 2.44275) (width 0.2) (layer "F.Cu") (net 43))
 (segment (start 99.13 3.89875) (end 97.674 2.44275) (width 0.2) (layer "F.Cu") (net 43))
 (segment (start 39.05725 2.44275) (end 24.5 17) (width 0.2) (layer "F.Cu") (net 43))
 (segment (start 18 17) (end 24.5 17) (width 0.2) (layer "B.Cu") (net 43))
 (segment (start 95.535 5.38375) (end 94.05 3.89875) (width 0.2) (layer "B.Cu") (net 4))
 (segment (start 101.183246 7) (end 99.566996 5.38375) (width 0.2) (layer "B.Cu") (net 4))
 (segment (start 126 7) (end 132.5 7) (width 0.2) (layer "B.Cu") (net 4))
 (segment (start 126 7) (end 101.183246 7) (width 0.2) (layer "B.Cu") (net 4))
 (segment (start 99.566996 5.38375) (end 95.535 5.38375) (width 0.2) (layer "B.Cu") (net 4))
 (segment (start 92.995 3.461754) (end 93.613004 2.84375) (width 0.2) (layer "B.Cu") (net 41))
 (segment (start 132.5 21.5) (end 126 21.5) (width 0.2) (layer "B.Cu") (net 41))
 (segment (start 92.995 4.335746) (end 92.995 3.461754) (width 0.2) (layer "B.Cu") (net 41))
 (segment (start 126 21.5) (end 124.699 22.801) (width 0.2) (layer "B.Cu") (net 41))
 (segment (start 95.535 6.875746) (end 95.535 6.001754) (width 0.2) (layer "B.Cu") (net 41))
 (segment (start 95.535 6.001754) (end 94.486996 4.95375) (width 0.2) (layer "B.Cu") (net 41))
 (segment (start 124.699 22.801) (end 111.460254 22.801) (width 0.2) (layer "B.Cu") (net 41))
 (segment (start 111.460254 22.801) (end 95.535 6.875746) (width 0.2) (layer "B.Cu") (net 41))
 (segment (start 95.535 2.84375) (end 96.59 3.89875) (width 0.2) (layer "B.Cu") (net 41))
 (segment (start 93.613004 4.95375) (end 92.995 4.335746) (width 0.2) (layer "B.Cu") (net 41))
 (segment (start 94.486996 4.95375) (end 93.613004 4.95375) (width 0.2) (layer "B.Cu") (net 41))
 (segment (start 93.613004 2.84375) (end 95.535 2.84375) (width 0.2) (layer "B.Cu") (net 41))
 (segment (start 17.461108 28.301) (end 25.308683 28.301) (width 0.2) (layer "B.Cu") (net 11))
 (segment (start 14.5 25.339892) (end 17.461108 28.301) (width 0.2) (layer "B.Cu") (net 11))
 (segment (start 47.726 5.883683) (end 47.726 5.316583) (width 0.2) (layer "B.Cu") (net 11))
 (segment (start 47.726 5.316583) (end 50.661333 2.38125) (width 0.2) (layer "B.Cu") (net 11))
 (segment (start 62.0525 2.38125) (end 63.57 3.89875) (width 0.2) (layer "B.Cu") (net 11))
 (segment (start 50.661333 2.38125) (end 62.0525 2.38125) (width 0.2) (layer "B.Cu") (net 11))
 (segment (start 14.5 21.5) (end 14.5 25.339892) (width 0.2) (layer "B.Cu") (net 11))
 (segment (start 25.308683 28.301) (end 47.726 5.883683) (width 0.2) (layer "B.Cu") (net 11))
 (segment (start 8 21.5) (end 14.5 21.5) (width 0.2) (layer "B.Cu") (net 11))
 (segment (start 65.055 4.765746) (end 65.673004 5.38375) (width 0.2) (layer "B.Cu") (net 12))
 (segment (start 65.055 3.891754) (end 65.055 4.765746) (width 0.2) (layer "B.Cu") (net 12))
 (segment (start 18 11.5) (end 24.5 11.5) (width 0.2) (layer "B.Cu") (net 12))
 (segment (start 16.699 10.199) (end 16.699 6.461108) (width 0.2) (layer "B.Cu") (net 12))
 (segment (start 65.673004 5.38375) (end 87.915 5.38375) (width 0.2) (layer "B.Cu") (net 12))
 (segment (start 87.915 5.38375) (end 88.97 6.43875) (width 0.2) (layer "B.Cu") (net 12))
 (segment (start 18 11.5) (end 16.699 10.199) (width 0.2) (layer "B.Cu") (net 12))
 (segment (start 16.699 6.461108) (end 21.179858 1.98025) (width 0.2) (layer "B.Cu") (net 12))
 (segment (start 63.143496 1.98025) (end 65.055 3.891754) (width 0.2) (layer "B.Cu") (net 12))
 (segment (start 21.179858 1.98025) (end 63.143496 1.98025) (width 0.2) (layer "B.Cu") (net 12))
 (segment (start 20.5425 56.73) (end 127.50075 56.73) (width 0.2) (layer "B.Cu") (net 8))
 (segment (start 18.8125 55) (end 20.5425 56.73) (width 0.2) (layer "B.Cu") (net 8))
 (segment (start 127.50075 56.73) (end 128.55575 57.785) (width 0.2) (layer "B.Cu") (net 8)))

